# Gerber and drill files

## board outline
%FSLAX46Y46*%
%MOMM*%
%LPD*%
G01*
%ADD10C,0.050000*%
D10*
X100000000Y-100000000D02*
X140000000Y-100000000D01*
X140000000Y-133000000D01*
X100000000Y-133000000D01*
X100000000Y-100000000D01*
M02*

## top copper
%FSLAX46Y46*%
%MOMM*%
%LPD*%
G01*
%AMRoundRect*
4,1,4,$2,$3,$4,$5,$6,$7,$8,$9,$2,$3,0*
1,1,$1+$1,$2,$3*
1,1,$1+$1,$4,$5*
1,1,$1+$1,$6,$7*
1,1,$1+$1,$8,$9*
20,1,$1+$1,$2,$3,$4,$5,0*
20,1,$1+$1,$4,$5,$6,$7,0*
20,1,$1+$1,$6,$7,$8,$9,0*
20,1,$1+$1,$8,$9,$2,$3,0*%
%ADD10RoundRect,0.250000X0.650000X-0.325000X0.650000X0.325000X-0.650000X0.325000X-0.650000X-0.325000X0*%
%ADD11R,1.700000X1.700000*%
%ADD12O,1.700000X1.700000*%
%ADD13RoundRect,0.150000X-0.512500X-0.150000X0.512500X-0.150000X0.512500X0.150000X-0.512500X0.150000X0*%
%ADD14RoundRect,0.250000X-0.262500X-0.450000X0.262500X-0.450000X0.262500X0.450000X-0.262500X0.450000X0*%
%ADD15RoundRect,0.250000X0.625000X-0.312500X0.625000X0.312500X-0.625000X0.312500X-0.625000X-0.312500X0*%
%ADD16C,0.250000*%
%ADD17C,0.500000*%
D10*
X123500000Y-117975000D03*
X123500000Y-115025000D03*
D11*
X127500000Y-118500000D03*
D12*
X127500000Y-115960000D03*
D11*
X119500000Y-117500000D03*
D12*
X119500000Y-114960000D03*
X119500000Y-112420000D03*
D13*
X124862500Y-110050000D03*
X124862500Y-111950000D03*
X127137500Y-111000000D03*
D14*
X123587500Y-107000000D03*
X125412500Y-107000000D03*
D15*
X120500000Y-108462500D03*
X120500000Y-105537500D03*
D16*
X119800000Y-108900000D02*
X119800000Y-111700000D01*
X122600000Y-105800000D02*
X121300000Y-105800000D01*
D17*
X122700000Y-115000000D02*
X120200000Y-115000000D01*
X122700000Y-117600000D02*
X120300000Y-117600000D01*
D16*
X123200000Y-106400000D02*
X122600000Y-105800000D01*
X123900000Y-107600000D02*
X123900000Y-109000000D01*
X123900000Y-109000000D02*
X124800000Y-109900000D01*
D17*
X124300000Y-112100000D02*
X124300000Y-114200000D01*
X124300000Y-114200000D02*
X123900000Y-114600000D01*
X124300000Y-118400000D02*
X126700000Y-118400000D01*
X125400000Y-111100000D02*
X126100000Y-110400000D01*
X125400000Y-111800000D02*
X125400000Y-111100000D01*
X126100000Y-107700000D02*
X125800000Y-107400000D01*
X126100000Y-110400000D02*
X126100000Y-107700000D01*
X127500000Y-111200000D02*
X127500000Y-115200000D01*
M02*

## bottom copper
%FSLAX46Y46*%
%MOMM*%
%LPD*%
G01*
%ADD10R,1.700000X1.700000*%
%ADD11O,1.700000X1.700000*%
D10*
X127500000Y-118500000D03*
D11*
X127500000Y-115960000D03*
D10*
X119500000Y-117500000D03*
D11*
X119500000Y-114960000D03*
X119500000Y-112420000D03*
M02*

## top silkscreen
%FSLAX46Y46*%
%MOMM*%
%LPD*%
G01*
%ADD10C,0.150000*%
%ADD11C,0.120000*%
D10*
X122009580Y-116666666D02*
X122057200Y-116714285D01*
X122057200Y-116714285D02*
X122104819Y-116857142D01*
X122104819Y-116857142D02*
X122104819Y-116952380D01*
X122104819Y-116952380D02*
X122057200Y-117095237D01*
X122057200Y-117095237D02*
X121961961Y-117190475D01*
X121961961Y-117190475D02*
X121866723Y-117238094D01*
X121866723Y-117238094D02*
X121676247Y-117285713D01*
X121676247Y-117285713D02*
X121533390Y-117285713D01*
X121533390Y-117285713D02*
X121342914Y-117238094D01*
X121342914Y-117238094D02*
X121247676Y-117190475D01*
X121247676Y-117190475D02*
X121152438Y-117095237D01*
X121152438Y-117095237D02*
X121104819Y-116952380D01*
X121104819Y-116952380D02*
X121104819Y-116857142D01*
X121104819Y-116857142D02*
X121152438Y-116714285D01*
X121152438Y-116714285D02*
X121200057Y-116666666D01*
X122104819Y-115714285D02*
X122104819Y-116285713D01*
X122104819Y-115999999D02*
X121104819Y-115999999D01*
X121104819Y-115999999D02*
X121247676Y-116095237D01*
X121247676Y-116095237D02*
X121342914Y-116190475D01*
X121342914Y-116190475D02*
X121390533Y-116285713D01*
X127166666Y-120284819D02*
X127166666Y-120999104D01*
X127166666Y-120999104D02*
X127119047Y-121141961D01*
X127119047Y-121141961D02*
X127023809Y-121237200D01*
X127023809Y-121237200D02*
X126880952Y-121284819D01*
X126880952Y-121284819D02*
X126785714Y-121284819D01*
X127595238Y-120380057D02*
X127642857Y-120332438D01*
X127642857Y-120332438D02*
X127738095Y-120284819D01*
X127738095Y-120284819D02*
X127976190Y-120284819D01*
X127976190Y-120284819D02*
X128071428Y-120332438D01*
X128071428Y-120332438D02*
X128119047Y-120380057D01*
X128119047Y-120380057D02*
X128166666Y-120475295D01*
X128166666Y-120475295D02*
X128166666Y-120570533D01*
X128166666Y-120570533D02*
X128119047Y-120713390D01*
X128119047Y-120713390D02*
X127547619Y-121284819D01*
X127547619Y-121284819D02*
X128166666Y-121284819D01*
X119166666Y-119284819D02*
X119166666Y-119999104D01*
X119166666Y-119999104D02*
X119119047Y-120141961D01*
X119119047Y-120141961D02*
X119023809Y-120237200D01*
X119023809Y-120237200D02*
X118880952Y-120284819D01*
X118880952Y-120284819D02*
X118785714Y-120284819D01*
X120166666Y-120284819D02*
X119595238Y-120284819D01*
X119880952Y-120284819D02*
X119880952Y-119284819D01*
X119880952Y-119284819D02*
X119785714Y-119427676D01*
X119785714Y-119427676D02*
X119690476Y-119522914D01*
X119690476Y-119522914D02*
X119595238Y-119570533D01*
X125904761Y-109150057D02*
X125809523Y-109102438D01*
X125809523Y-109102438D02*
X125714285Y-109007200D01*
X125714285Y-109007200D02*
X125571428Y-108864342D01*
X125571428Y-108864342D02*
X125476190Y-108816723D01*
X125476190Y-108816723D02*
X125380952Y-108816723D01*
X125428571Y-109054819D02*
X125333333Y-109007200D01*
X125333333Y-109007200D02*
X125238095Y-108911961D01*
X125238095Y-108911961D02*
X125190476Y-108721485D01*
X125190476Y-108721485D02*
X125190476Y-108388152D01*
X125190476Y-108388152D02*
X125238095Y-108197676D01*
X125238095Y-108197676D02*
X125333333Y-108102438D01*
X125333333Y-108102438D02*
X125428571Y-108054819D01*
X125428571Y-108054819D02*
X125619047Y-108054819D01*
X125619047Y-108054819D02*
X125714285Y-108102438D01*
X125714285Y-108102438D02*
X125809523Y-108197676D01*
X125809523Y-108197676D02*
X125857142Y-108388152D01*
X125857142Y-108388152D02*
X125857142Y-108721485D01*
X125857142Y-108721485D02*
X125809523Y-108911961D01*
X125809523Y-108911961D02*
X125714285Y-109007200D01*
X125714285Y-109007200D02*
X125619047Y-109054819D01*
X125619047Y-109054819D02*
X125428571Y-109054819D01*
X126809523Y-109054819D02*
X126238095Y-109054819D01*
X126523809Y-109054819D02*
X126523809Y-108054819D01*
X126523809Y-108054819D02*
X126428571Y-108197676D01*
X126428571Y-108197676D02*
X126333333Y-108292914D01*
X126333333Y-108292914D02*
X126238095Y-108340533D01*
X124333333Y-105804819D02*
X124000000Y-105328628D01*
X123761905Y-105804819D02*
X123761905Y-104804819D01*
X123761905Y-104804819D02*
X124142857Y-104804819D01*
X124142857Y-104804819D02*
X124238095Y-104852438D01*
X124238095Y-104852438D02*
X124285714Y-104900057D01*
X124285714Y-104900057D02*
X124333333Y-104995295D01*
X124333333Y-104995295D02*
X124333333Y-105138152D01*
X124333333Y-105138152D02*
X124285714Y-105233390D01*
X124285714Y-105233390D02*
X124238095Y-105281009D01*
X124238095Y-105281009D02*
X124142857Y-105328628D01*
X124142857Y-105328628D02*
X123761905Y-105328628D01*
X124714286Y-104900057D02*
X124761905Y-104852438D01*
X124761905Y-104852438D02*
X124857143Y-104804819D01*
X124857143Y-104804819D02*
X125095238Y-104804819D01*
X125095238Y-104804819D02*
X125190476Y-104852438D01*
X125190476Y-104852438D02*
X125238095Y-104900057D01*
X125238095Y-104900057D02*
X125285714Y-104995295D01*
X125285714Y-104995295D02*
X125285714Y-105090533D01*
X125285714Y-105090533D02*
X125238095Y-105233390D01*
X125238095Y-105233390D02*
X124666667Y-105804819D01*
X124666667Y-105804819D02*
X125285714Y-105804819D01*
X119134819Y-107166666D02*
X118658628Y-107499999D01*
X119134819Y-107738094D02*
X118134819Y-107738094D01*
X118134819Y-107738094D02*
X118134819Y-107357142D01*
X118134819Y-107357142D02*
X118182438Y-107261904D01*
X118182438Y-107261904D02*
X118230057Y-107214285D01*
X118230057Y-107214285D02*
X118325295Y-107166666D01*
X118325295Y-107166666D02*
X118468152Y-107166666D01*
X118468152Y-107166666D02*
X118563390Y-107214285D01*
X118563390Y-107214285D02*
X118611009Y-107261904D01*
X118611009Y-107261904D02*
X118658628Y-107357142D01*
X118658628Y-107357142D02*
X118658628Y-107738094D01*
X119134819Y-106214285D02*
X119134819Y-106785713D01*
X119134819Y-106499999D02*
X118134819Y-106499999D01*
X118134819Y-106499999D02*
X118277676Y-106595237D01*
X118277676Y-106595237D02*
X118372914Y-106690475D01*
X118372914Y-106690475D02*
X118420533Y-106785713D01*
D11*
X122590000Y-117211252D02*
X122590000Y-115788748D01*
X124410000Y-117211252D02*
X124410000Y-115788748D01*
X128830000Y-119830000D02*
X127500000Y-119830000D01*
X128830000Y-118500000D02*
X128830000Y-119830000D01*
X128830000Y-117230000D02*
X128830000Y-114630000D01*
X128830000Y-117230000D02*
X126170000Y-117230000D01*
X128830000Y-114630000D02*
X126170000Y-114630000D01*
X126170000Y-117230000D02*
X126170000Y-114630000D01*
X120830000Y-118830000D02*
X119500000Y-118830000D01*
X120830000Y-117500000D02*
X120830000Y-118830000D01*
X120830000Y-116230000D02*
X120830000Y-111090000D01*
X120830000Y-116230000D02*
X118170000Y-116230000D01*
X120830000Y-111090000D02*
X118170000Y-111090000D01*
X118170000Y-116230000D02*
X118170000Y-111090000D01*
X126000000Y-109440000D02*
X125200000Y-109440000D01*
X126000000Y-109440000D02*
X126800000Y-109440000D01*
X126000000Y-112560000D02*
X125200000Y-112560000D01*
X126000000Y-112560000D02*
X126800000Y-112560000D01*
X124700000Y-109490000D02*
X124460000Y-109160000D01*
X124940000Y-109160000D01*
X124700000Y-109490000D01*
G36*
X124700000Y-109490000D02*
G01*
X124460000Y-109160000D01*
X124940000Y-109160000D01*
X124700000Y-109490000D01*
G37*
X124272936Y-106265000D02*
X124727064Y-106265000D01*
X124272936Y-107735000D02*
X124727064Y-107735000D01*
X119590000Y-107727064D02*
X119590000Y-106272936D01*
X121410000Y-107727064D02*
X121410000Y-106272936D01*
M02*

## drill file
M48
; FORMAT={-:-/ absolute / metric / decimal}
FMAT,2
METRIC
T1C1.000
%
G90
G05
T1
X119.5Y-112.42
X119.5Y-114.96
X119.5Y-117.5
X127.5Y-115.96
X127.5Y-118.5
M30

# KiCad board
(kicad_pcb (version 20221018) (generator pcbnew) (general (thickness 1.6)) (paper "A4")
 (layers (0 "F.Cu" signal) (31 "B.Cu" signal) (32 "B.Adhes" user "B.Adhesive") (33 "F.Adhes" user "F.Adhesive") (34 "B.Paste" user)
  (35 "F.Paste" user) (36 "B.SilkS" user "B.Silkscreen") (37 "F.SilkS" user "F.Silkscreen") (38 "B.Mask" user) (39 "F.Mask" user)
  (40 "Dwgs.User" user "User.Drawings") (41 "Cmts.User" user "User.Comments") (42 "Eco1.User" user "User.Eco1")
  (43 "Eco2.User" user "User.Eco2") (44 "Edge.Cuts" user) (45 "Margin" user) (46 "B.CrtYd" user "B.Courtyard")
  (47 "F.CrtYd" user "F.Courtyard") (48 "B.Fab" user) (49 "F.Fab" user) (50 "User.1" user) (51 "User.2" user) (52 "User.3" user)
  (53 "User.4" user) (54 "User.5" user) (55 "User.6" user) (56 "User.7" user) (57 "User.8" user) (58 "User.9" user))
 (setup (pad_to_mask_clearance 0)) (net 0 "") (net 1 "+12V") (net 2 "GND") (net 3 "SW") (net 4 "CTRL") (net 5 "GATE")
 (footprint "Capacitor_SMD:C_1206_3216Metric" (layer "F.Cu") (at 123.5 116.5 90)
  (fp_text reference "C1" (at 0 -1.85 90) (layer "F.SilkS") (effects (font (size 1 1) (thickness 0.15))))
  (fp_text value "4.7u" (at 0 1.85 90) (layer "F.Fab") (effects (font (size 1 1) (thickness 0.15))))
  (fp_line (start -0.711252 -0.91) (end 0.711252 -0.91) (stroke (width 0.12) (type solid)) (layer "F.SilkS"))
  (fp_line (start -0.711252 0.91) (end 0.711252 0.91) (stroke (width 0.12) (type solid)) (layer "F.SilkS"))
  (pad "1" smd roundrect (at -1.475 0 90) (size 1.15 1.8) (layers "F.Cu" "F.Paste" "F.Mask") (roundrect_rratio 0.217391) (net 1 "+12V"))
  (pad "2" smd roundrect (at 1.475 0 90) (size 1.15 1.8) (layers "F.Cu" "F.Paste" "F.Mask") (roundrect_rratio 0.217391) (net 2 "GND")))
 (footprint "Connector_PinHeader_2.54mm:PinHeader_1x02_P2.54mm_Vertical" (layer "F.Cu") (at 127.5 118.5 180)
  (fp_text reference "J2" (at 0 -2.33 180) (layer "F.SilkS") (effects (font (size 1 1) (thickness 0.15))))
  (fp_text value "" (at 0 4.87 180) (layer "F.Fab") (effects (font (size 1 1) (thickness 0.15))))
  (fp_line (start -1.33 -1.33) (end 0 -1.33) (stroke (width 0.12) (type solid)) (layer "F.SilkS"))
  (fp_line (start -1.33 0) (end -1.33 -1.33) (stroke (width 0.12) (type solid)) (layer "F.SilkS"))
  (fp_line (start -1.33 1.27) (end -1.33 3.87) (stroke (width 0.12) (type solid)) (layer "F.SilkS"))
  (fp_line (start -1.33 1.27) (end 1.33 1.27) (stroke (width 0.12) (type solid)) (layer "F.SilkS"))
  (fp_line (start -1.33 3.87) (end 1.33 3.87) (stroke (width 0.12) (type solid)) (layer "F.SilkS"))
  (fp_line (start 1.33 1.27) (end 1.33 3.87) (stroke (width 0.12) (type solid)) (layer "F.SilkS"))
  (pad "1" thru_hole rect (at 0 0 180) (size 1.7 1.7) (drill 1) (layers "*.Cu" "*.Mask") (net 1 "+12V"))
  (pad "2" thru_hole oval (at 0 2.54 180) (size 1.7 1.7) (drill 1) (layers "*.Cu" "*.Mask") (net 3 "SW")))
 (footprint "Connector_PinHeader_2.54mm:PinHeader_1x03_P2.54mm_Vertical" (layer "F.Cu") (at 119.5 117.5 180)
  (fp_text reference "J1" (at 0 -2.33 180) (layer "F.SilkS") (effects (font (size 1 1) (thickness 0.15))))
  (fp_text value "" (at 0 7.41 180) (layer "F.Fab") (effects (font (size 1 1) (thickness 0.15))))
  (fp_line (start -1.33 -1.33) (end 0 -1.33) (stroke (width 0.12) (type solid)) (layer "F.SilkS"))
  (fp_line (start -1.33 0) (end -1.33 -1.33) (stroke (width 0.12) (type solid)) (layer "F.SilkS"))
  (fp_line (start -1.33 1.27) (end -1.33 6.41) (stroke (width 0.12) (type solid)) (layer "F.SilkS"))
  (fp_line (start -1.33 1.27) (end 1.33 1.27) (stroke (width 0.12) (type solid)) (layer "F.SilkS"))
  (fp_line (start -1.33 6.41) (end 1.33 6.41) (stroke (width 0.12) (type solid)) (layer "F.SilkS"))
  (fp_line (start 1.33 1.27) (end 1.33 6.41) (stroke (width 0.12) (type solid)) (layer "F.SilkS"))
  (pad "1" thru_hole rect (at 0 0 180) (size 1.7 1.7) (drill 1) (layers "*.Cu" "*.Mask") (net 1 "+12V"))
  (pad "2" thru_hole oval (at 0 2.54 180) (size 1.7 1.7) (drill 1) (layers "*.Cu" "*.Mask") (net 2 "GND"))
  (pad "3" thru_hole oval (at 0 5.08 180) (size 1.7 1.7) (drill 1) (layers "*.Cu" "*.Mask") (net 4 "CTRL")))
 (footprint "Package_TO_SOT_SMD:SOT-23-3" (layer "F.Cu") (at 126 111)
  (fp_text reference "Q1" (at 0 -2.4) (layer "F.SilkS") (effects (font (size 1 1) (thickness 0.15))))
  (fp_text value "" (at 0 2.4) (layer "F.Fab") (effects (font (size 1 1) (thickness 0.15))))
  (fp_line (start 0 -1.56) (end -0.8 -1.56) (stroke (width 0.12) (type solid)) (layer "F.SilkS"))
  (fp_line (start 0 -1.56) (end 0.8 -1.56) (stroke (width 0.12) (type solid)) (layer "F.SilkS"))
  (fp_line (start 0 1.56) (end -0.8 1.56) (stroke (width 0.12) (type solid)) (layer "F.SilkS"))
  (fp_line (start 0 1.56) (end 0.8 1.56) (stroke (width 0.12) (type solid)) (layer "F.SilkS"))
  (fp_poly
   (pts (xy -1.3 -1.51) (xy -1.54 -1.84) (xy -1.06 -1.84) (xy -1.3 -1.51)) (stroke (width 0.12) (type solid)) (fill solid) (layer "F.SilkS"))
  (pad "1" smd roundrect (at -1.1375 -0.95) (size 1.325 0.6) (layers "F.Cu" "F.Paste" "F.Mask") (roundrect_rratio 0.25) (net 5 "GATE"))
  (pad "2" smd roundrect (at -1.1375 0.95) (size 1.325 0.6) (layers "F.Cu" "F.Paste" "F.Mask") (roundrect_rratio 0.25) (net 2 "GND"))
  (pad "3" smd roundrect (at 1.1375 0) (size 1.325 0.6) (layers "F.Cu" "F.Paste" "F.Mask") (roundrect_rratio 0.25) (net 3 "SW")))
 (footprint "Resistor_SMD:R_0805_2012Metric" (layer "F.Cu") (at 124.5 107)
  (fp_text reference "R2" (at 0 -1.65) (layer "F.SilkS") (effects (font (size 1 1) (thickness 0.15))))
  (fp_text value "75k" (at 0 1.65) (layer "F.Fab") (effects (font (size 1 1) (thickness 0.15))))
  (fp_line (start -0.227064 -0.735) (end 0.227064 -0.735) (stroke (width 0.12) (type solid)) (layer "F.SilkS"))
  (fp_line (start -0.227064 0.735) (end 0.227064 0.735) (stroke (width 0.12) (type solid)) (layer "F.SilkS"))
  (pad "1" smd roundrect (at -0.9125 0) (size 1.025 1.4) (layers "F.Cu" "F.Paste" "F.Mask") (roundrect_rratio 0.243902) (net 5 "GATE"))
  (pad "2" smd roundrect (at 0.9125 0) (size 1.025 1.4) (layers "F.Cu" "F.Paste" "F.Mask") (roundrect_rratio 0.243902) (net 2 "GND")))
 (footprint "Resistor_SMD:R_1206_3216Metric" (layer "F.Cu") (at 120.5 107 90)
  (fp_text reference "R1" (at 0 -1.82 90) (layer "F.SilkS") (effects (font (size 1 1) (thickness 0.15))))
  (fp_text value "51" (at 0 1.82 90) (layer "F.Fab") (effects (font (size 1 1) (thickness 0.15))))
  (fp_line (start -0.727064 -0.91) (end 0.727064 -0.91) (stroke (width 0.12) (type solid)) (layer "F.SilkS"))
  (fp_line (start -0.727064 0.91) (end 0.727064 0.91) (stroke (width 0.12) (type solid)) (layer "F.SilkS"))
  (pad "1" smd roundrect (at -1.4625 0 90) (size 1.125 1.75) (layers "F.Cu" "F.Paste" "F.Mask") (roundrect_rratio 0.222222) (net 4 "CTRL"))
  (pad "2" smd roundrect (at 1.4625 0 90) (size 1.125 1.75) (layers "F.Cu" "F.Paste" "F.Mask") (roundrect_rratio 0.222222) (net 5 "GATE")))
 (gr_rect (start 100 100) (end 140 133) (stroke (width 0.05) (type default)) (fill none) (layer "Edge.Cuts"))
 (segment (start 119.8 108.9) (end 119.8 111.7) (width 0.25) (layer "F.Cu") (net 4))
 (segment (start 122.6 105.8) (end 121.3 105.8) (width 0.25) (layer "F.Cu") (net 5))
 (segment (start 122.7 115) (end 120.2 115) (width 0.5) (layer "F.Cu") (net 2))
 (segment (start 122.7 117.6) (end 120.3 117.6) (width 0.5) (layer "F.Cu") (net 1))
 (segment (start 123.2 106.4) (end 122.6 105.8) (width 0.25) (layer "F.Cu") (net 5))
 (segment (start 123.9 107.6) (end 123.9 109) (width 0.25) (layer "F.Cu") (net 5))
 (segment (start 123.9 109) (end 124.8 109.9) (width 0.25) (layer "F.Cu") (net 5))
 (segment (start 124.3 112.1) (end 124.3 114.2) (width 0.5) (layer "F.Cu") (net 2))
 (segment (start 124.3 114.2) (end 123.9 114.6) (width 0.5) (layer "F.Cu") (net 2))
 (segment (start 124.3 118.4) (end 126.7 118.4) (width 0.5) (layer "F.Cu") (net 1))
 (segment (start 125.4 111.1) (end 126.1 110.4) (width 0.5) (layer "F.Cu") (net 2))
 (segment (start 125.4 111.8) (end 125.4 111.1) (width 0.5) (layer "F.Cu") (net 2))
 (segment (start 126.1 107.7) (end 125.8 107.4) (width 0.5) (layer "F.Cu") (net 2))
 (segment (start 126.1 110.4) (end 126.1 107.7) (width 0.5) (layer "F.Cu") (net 2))
 (segment (start 127.5 111.2) (end 127.5 115.2) (width 0.5) (layer "F.Cu") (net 3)))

